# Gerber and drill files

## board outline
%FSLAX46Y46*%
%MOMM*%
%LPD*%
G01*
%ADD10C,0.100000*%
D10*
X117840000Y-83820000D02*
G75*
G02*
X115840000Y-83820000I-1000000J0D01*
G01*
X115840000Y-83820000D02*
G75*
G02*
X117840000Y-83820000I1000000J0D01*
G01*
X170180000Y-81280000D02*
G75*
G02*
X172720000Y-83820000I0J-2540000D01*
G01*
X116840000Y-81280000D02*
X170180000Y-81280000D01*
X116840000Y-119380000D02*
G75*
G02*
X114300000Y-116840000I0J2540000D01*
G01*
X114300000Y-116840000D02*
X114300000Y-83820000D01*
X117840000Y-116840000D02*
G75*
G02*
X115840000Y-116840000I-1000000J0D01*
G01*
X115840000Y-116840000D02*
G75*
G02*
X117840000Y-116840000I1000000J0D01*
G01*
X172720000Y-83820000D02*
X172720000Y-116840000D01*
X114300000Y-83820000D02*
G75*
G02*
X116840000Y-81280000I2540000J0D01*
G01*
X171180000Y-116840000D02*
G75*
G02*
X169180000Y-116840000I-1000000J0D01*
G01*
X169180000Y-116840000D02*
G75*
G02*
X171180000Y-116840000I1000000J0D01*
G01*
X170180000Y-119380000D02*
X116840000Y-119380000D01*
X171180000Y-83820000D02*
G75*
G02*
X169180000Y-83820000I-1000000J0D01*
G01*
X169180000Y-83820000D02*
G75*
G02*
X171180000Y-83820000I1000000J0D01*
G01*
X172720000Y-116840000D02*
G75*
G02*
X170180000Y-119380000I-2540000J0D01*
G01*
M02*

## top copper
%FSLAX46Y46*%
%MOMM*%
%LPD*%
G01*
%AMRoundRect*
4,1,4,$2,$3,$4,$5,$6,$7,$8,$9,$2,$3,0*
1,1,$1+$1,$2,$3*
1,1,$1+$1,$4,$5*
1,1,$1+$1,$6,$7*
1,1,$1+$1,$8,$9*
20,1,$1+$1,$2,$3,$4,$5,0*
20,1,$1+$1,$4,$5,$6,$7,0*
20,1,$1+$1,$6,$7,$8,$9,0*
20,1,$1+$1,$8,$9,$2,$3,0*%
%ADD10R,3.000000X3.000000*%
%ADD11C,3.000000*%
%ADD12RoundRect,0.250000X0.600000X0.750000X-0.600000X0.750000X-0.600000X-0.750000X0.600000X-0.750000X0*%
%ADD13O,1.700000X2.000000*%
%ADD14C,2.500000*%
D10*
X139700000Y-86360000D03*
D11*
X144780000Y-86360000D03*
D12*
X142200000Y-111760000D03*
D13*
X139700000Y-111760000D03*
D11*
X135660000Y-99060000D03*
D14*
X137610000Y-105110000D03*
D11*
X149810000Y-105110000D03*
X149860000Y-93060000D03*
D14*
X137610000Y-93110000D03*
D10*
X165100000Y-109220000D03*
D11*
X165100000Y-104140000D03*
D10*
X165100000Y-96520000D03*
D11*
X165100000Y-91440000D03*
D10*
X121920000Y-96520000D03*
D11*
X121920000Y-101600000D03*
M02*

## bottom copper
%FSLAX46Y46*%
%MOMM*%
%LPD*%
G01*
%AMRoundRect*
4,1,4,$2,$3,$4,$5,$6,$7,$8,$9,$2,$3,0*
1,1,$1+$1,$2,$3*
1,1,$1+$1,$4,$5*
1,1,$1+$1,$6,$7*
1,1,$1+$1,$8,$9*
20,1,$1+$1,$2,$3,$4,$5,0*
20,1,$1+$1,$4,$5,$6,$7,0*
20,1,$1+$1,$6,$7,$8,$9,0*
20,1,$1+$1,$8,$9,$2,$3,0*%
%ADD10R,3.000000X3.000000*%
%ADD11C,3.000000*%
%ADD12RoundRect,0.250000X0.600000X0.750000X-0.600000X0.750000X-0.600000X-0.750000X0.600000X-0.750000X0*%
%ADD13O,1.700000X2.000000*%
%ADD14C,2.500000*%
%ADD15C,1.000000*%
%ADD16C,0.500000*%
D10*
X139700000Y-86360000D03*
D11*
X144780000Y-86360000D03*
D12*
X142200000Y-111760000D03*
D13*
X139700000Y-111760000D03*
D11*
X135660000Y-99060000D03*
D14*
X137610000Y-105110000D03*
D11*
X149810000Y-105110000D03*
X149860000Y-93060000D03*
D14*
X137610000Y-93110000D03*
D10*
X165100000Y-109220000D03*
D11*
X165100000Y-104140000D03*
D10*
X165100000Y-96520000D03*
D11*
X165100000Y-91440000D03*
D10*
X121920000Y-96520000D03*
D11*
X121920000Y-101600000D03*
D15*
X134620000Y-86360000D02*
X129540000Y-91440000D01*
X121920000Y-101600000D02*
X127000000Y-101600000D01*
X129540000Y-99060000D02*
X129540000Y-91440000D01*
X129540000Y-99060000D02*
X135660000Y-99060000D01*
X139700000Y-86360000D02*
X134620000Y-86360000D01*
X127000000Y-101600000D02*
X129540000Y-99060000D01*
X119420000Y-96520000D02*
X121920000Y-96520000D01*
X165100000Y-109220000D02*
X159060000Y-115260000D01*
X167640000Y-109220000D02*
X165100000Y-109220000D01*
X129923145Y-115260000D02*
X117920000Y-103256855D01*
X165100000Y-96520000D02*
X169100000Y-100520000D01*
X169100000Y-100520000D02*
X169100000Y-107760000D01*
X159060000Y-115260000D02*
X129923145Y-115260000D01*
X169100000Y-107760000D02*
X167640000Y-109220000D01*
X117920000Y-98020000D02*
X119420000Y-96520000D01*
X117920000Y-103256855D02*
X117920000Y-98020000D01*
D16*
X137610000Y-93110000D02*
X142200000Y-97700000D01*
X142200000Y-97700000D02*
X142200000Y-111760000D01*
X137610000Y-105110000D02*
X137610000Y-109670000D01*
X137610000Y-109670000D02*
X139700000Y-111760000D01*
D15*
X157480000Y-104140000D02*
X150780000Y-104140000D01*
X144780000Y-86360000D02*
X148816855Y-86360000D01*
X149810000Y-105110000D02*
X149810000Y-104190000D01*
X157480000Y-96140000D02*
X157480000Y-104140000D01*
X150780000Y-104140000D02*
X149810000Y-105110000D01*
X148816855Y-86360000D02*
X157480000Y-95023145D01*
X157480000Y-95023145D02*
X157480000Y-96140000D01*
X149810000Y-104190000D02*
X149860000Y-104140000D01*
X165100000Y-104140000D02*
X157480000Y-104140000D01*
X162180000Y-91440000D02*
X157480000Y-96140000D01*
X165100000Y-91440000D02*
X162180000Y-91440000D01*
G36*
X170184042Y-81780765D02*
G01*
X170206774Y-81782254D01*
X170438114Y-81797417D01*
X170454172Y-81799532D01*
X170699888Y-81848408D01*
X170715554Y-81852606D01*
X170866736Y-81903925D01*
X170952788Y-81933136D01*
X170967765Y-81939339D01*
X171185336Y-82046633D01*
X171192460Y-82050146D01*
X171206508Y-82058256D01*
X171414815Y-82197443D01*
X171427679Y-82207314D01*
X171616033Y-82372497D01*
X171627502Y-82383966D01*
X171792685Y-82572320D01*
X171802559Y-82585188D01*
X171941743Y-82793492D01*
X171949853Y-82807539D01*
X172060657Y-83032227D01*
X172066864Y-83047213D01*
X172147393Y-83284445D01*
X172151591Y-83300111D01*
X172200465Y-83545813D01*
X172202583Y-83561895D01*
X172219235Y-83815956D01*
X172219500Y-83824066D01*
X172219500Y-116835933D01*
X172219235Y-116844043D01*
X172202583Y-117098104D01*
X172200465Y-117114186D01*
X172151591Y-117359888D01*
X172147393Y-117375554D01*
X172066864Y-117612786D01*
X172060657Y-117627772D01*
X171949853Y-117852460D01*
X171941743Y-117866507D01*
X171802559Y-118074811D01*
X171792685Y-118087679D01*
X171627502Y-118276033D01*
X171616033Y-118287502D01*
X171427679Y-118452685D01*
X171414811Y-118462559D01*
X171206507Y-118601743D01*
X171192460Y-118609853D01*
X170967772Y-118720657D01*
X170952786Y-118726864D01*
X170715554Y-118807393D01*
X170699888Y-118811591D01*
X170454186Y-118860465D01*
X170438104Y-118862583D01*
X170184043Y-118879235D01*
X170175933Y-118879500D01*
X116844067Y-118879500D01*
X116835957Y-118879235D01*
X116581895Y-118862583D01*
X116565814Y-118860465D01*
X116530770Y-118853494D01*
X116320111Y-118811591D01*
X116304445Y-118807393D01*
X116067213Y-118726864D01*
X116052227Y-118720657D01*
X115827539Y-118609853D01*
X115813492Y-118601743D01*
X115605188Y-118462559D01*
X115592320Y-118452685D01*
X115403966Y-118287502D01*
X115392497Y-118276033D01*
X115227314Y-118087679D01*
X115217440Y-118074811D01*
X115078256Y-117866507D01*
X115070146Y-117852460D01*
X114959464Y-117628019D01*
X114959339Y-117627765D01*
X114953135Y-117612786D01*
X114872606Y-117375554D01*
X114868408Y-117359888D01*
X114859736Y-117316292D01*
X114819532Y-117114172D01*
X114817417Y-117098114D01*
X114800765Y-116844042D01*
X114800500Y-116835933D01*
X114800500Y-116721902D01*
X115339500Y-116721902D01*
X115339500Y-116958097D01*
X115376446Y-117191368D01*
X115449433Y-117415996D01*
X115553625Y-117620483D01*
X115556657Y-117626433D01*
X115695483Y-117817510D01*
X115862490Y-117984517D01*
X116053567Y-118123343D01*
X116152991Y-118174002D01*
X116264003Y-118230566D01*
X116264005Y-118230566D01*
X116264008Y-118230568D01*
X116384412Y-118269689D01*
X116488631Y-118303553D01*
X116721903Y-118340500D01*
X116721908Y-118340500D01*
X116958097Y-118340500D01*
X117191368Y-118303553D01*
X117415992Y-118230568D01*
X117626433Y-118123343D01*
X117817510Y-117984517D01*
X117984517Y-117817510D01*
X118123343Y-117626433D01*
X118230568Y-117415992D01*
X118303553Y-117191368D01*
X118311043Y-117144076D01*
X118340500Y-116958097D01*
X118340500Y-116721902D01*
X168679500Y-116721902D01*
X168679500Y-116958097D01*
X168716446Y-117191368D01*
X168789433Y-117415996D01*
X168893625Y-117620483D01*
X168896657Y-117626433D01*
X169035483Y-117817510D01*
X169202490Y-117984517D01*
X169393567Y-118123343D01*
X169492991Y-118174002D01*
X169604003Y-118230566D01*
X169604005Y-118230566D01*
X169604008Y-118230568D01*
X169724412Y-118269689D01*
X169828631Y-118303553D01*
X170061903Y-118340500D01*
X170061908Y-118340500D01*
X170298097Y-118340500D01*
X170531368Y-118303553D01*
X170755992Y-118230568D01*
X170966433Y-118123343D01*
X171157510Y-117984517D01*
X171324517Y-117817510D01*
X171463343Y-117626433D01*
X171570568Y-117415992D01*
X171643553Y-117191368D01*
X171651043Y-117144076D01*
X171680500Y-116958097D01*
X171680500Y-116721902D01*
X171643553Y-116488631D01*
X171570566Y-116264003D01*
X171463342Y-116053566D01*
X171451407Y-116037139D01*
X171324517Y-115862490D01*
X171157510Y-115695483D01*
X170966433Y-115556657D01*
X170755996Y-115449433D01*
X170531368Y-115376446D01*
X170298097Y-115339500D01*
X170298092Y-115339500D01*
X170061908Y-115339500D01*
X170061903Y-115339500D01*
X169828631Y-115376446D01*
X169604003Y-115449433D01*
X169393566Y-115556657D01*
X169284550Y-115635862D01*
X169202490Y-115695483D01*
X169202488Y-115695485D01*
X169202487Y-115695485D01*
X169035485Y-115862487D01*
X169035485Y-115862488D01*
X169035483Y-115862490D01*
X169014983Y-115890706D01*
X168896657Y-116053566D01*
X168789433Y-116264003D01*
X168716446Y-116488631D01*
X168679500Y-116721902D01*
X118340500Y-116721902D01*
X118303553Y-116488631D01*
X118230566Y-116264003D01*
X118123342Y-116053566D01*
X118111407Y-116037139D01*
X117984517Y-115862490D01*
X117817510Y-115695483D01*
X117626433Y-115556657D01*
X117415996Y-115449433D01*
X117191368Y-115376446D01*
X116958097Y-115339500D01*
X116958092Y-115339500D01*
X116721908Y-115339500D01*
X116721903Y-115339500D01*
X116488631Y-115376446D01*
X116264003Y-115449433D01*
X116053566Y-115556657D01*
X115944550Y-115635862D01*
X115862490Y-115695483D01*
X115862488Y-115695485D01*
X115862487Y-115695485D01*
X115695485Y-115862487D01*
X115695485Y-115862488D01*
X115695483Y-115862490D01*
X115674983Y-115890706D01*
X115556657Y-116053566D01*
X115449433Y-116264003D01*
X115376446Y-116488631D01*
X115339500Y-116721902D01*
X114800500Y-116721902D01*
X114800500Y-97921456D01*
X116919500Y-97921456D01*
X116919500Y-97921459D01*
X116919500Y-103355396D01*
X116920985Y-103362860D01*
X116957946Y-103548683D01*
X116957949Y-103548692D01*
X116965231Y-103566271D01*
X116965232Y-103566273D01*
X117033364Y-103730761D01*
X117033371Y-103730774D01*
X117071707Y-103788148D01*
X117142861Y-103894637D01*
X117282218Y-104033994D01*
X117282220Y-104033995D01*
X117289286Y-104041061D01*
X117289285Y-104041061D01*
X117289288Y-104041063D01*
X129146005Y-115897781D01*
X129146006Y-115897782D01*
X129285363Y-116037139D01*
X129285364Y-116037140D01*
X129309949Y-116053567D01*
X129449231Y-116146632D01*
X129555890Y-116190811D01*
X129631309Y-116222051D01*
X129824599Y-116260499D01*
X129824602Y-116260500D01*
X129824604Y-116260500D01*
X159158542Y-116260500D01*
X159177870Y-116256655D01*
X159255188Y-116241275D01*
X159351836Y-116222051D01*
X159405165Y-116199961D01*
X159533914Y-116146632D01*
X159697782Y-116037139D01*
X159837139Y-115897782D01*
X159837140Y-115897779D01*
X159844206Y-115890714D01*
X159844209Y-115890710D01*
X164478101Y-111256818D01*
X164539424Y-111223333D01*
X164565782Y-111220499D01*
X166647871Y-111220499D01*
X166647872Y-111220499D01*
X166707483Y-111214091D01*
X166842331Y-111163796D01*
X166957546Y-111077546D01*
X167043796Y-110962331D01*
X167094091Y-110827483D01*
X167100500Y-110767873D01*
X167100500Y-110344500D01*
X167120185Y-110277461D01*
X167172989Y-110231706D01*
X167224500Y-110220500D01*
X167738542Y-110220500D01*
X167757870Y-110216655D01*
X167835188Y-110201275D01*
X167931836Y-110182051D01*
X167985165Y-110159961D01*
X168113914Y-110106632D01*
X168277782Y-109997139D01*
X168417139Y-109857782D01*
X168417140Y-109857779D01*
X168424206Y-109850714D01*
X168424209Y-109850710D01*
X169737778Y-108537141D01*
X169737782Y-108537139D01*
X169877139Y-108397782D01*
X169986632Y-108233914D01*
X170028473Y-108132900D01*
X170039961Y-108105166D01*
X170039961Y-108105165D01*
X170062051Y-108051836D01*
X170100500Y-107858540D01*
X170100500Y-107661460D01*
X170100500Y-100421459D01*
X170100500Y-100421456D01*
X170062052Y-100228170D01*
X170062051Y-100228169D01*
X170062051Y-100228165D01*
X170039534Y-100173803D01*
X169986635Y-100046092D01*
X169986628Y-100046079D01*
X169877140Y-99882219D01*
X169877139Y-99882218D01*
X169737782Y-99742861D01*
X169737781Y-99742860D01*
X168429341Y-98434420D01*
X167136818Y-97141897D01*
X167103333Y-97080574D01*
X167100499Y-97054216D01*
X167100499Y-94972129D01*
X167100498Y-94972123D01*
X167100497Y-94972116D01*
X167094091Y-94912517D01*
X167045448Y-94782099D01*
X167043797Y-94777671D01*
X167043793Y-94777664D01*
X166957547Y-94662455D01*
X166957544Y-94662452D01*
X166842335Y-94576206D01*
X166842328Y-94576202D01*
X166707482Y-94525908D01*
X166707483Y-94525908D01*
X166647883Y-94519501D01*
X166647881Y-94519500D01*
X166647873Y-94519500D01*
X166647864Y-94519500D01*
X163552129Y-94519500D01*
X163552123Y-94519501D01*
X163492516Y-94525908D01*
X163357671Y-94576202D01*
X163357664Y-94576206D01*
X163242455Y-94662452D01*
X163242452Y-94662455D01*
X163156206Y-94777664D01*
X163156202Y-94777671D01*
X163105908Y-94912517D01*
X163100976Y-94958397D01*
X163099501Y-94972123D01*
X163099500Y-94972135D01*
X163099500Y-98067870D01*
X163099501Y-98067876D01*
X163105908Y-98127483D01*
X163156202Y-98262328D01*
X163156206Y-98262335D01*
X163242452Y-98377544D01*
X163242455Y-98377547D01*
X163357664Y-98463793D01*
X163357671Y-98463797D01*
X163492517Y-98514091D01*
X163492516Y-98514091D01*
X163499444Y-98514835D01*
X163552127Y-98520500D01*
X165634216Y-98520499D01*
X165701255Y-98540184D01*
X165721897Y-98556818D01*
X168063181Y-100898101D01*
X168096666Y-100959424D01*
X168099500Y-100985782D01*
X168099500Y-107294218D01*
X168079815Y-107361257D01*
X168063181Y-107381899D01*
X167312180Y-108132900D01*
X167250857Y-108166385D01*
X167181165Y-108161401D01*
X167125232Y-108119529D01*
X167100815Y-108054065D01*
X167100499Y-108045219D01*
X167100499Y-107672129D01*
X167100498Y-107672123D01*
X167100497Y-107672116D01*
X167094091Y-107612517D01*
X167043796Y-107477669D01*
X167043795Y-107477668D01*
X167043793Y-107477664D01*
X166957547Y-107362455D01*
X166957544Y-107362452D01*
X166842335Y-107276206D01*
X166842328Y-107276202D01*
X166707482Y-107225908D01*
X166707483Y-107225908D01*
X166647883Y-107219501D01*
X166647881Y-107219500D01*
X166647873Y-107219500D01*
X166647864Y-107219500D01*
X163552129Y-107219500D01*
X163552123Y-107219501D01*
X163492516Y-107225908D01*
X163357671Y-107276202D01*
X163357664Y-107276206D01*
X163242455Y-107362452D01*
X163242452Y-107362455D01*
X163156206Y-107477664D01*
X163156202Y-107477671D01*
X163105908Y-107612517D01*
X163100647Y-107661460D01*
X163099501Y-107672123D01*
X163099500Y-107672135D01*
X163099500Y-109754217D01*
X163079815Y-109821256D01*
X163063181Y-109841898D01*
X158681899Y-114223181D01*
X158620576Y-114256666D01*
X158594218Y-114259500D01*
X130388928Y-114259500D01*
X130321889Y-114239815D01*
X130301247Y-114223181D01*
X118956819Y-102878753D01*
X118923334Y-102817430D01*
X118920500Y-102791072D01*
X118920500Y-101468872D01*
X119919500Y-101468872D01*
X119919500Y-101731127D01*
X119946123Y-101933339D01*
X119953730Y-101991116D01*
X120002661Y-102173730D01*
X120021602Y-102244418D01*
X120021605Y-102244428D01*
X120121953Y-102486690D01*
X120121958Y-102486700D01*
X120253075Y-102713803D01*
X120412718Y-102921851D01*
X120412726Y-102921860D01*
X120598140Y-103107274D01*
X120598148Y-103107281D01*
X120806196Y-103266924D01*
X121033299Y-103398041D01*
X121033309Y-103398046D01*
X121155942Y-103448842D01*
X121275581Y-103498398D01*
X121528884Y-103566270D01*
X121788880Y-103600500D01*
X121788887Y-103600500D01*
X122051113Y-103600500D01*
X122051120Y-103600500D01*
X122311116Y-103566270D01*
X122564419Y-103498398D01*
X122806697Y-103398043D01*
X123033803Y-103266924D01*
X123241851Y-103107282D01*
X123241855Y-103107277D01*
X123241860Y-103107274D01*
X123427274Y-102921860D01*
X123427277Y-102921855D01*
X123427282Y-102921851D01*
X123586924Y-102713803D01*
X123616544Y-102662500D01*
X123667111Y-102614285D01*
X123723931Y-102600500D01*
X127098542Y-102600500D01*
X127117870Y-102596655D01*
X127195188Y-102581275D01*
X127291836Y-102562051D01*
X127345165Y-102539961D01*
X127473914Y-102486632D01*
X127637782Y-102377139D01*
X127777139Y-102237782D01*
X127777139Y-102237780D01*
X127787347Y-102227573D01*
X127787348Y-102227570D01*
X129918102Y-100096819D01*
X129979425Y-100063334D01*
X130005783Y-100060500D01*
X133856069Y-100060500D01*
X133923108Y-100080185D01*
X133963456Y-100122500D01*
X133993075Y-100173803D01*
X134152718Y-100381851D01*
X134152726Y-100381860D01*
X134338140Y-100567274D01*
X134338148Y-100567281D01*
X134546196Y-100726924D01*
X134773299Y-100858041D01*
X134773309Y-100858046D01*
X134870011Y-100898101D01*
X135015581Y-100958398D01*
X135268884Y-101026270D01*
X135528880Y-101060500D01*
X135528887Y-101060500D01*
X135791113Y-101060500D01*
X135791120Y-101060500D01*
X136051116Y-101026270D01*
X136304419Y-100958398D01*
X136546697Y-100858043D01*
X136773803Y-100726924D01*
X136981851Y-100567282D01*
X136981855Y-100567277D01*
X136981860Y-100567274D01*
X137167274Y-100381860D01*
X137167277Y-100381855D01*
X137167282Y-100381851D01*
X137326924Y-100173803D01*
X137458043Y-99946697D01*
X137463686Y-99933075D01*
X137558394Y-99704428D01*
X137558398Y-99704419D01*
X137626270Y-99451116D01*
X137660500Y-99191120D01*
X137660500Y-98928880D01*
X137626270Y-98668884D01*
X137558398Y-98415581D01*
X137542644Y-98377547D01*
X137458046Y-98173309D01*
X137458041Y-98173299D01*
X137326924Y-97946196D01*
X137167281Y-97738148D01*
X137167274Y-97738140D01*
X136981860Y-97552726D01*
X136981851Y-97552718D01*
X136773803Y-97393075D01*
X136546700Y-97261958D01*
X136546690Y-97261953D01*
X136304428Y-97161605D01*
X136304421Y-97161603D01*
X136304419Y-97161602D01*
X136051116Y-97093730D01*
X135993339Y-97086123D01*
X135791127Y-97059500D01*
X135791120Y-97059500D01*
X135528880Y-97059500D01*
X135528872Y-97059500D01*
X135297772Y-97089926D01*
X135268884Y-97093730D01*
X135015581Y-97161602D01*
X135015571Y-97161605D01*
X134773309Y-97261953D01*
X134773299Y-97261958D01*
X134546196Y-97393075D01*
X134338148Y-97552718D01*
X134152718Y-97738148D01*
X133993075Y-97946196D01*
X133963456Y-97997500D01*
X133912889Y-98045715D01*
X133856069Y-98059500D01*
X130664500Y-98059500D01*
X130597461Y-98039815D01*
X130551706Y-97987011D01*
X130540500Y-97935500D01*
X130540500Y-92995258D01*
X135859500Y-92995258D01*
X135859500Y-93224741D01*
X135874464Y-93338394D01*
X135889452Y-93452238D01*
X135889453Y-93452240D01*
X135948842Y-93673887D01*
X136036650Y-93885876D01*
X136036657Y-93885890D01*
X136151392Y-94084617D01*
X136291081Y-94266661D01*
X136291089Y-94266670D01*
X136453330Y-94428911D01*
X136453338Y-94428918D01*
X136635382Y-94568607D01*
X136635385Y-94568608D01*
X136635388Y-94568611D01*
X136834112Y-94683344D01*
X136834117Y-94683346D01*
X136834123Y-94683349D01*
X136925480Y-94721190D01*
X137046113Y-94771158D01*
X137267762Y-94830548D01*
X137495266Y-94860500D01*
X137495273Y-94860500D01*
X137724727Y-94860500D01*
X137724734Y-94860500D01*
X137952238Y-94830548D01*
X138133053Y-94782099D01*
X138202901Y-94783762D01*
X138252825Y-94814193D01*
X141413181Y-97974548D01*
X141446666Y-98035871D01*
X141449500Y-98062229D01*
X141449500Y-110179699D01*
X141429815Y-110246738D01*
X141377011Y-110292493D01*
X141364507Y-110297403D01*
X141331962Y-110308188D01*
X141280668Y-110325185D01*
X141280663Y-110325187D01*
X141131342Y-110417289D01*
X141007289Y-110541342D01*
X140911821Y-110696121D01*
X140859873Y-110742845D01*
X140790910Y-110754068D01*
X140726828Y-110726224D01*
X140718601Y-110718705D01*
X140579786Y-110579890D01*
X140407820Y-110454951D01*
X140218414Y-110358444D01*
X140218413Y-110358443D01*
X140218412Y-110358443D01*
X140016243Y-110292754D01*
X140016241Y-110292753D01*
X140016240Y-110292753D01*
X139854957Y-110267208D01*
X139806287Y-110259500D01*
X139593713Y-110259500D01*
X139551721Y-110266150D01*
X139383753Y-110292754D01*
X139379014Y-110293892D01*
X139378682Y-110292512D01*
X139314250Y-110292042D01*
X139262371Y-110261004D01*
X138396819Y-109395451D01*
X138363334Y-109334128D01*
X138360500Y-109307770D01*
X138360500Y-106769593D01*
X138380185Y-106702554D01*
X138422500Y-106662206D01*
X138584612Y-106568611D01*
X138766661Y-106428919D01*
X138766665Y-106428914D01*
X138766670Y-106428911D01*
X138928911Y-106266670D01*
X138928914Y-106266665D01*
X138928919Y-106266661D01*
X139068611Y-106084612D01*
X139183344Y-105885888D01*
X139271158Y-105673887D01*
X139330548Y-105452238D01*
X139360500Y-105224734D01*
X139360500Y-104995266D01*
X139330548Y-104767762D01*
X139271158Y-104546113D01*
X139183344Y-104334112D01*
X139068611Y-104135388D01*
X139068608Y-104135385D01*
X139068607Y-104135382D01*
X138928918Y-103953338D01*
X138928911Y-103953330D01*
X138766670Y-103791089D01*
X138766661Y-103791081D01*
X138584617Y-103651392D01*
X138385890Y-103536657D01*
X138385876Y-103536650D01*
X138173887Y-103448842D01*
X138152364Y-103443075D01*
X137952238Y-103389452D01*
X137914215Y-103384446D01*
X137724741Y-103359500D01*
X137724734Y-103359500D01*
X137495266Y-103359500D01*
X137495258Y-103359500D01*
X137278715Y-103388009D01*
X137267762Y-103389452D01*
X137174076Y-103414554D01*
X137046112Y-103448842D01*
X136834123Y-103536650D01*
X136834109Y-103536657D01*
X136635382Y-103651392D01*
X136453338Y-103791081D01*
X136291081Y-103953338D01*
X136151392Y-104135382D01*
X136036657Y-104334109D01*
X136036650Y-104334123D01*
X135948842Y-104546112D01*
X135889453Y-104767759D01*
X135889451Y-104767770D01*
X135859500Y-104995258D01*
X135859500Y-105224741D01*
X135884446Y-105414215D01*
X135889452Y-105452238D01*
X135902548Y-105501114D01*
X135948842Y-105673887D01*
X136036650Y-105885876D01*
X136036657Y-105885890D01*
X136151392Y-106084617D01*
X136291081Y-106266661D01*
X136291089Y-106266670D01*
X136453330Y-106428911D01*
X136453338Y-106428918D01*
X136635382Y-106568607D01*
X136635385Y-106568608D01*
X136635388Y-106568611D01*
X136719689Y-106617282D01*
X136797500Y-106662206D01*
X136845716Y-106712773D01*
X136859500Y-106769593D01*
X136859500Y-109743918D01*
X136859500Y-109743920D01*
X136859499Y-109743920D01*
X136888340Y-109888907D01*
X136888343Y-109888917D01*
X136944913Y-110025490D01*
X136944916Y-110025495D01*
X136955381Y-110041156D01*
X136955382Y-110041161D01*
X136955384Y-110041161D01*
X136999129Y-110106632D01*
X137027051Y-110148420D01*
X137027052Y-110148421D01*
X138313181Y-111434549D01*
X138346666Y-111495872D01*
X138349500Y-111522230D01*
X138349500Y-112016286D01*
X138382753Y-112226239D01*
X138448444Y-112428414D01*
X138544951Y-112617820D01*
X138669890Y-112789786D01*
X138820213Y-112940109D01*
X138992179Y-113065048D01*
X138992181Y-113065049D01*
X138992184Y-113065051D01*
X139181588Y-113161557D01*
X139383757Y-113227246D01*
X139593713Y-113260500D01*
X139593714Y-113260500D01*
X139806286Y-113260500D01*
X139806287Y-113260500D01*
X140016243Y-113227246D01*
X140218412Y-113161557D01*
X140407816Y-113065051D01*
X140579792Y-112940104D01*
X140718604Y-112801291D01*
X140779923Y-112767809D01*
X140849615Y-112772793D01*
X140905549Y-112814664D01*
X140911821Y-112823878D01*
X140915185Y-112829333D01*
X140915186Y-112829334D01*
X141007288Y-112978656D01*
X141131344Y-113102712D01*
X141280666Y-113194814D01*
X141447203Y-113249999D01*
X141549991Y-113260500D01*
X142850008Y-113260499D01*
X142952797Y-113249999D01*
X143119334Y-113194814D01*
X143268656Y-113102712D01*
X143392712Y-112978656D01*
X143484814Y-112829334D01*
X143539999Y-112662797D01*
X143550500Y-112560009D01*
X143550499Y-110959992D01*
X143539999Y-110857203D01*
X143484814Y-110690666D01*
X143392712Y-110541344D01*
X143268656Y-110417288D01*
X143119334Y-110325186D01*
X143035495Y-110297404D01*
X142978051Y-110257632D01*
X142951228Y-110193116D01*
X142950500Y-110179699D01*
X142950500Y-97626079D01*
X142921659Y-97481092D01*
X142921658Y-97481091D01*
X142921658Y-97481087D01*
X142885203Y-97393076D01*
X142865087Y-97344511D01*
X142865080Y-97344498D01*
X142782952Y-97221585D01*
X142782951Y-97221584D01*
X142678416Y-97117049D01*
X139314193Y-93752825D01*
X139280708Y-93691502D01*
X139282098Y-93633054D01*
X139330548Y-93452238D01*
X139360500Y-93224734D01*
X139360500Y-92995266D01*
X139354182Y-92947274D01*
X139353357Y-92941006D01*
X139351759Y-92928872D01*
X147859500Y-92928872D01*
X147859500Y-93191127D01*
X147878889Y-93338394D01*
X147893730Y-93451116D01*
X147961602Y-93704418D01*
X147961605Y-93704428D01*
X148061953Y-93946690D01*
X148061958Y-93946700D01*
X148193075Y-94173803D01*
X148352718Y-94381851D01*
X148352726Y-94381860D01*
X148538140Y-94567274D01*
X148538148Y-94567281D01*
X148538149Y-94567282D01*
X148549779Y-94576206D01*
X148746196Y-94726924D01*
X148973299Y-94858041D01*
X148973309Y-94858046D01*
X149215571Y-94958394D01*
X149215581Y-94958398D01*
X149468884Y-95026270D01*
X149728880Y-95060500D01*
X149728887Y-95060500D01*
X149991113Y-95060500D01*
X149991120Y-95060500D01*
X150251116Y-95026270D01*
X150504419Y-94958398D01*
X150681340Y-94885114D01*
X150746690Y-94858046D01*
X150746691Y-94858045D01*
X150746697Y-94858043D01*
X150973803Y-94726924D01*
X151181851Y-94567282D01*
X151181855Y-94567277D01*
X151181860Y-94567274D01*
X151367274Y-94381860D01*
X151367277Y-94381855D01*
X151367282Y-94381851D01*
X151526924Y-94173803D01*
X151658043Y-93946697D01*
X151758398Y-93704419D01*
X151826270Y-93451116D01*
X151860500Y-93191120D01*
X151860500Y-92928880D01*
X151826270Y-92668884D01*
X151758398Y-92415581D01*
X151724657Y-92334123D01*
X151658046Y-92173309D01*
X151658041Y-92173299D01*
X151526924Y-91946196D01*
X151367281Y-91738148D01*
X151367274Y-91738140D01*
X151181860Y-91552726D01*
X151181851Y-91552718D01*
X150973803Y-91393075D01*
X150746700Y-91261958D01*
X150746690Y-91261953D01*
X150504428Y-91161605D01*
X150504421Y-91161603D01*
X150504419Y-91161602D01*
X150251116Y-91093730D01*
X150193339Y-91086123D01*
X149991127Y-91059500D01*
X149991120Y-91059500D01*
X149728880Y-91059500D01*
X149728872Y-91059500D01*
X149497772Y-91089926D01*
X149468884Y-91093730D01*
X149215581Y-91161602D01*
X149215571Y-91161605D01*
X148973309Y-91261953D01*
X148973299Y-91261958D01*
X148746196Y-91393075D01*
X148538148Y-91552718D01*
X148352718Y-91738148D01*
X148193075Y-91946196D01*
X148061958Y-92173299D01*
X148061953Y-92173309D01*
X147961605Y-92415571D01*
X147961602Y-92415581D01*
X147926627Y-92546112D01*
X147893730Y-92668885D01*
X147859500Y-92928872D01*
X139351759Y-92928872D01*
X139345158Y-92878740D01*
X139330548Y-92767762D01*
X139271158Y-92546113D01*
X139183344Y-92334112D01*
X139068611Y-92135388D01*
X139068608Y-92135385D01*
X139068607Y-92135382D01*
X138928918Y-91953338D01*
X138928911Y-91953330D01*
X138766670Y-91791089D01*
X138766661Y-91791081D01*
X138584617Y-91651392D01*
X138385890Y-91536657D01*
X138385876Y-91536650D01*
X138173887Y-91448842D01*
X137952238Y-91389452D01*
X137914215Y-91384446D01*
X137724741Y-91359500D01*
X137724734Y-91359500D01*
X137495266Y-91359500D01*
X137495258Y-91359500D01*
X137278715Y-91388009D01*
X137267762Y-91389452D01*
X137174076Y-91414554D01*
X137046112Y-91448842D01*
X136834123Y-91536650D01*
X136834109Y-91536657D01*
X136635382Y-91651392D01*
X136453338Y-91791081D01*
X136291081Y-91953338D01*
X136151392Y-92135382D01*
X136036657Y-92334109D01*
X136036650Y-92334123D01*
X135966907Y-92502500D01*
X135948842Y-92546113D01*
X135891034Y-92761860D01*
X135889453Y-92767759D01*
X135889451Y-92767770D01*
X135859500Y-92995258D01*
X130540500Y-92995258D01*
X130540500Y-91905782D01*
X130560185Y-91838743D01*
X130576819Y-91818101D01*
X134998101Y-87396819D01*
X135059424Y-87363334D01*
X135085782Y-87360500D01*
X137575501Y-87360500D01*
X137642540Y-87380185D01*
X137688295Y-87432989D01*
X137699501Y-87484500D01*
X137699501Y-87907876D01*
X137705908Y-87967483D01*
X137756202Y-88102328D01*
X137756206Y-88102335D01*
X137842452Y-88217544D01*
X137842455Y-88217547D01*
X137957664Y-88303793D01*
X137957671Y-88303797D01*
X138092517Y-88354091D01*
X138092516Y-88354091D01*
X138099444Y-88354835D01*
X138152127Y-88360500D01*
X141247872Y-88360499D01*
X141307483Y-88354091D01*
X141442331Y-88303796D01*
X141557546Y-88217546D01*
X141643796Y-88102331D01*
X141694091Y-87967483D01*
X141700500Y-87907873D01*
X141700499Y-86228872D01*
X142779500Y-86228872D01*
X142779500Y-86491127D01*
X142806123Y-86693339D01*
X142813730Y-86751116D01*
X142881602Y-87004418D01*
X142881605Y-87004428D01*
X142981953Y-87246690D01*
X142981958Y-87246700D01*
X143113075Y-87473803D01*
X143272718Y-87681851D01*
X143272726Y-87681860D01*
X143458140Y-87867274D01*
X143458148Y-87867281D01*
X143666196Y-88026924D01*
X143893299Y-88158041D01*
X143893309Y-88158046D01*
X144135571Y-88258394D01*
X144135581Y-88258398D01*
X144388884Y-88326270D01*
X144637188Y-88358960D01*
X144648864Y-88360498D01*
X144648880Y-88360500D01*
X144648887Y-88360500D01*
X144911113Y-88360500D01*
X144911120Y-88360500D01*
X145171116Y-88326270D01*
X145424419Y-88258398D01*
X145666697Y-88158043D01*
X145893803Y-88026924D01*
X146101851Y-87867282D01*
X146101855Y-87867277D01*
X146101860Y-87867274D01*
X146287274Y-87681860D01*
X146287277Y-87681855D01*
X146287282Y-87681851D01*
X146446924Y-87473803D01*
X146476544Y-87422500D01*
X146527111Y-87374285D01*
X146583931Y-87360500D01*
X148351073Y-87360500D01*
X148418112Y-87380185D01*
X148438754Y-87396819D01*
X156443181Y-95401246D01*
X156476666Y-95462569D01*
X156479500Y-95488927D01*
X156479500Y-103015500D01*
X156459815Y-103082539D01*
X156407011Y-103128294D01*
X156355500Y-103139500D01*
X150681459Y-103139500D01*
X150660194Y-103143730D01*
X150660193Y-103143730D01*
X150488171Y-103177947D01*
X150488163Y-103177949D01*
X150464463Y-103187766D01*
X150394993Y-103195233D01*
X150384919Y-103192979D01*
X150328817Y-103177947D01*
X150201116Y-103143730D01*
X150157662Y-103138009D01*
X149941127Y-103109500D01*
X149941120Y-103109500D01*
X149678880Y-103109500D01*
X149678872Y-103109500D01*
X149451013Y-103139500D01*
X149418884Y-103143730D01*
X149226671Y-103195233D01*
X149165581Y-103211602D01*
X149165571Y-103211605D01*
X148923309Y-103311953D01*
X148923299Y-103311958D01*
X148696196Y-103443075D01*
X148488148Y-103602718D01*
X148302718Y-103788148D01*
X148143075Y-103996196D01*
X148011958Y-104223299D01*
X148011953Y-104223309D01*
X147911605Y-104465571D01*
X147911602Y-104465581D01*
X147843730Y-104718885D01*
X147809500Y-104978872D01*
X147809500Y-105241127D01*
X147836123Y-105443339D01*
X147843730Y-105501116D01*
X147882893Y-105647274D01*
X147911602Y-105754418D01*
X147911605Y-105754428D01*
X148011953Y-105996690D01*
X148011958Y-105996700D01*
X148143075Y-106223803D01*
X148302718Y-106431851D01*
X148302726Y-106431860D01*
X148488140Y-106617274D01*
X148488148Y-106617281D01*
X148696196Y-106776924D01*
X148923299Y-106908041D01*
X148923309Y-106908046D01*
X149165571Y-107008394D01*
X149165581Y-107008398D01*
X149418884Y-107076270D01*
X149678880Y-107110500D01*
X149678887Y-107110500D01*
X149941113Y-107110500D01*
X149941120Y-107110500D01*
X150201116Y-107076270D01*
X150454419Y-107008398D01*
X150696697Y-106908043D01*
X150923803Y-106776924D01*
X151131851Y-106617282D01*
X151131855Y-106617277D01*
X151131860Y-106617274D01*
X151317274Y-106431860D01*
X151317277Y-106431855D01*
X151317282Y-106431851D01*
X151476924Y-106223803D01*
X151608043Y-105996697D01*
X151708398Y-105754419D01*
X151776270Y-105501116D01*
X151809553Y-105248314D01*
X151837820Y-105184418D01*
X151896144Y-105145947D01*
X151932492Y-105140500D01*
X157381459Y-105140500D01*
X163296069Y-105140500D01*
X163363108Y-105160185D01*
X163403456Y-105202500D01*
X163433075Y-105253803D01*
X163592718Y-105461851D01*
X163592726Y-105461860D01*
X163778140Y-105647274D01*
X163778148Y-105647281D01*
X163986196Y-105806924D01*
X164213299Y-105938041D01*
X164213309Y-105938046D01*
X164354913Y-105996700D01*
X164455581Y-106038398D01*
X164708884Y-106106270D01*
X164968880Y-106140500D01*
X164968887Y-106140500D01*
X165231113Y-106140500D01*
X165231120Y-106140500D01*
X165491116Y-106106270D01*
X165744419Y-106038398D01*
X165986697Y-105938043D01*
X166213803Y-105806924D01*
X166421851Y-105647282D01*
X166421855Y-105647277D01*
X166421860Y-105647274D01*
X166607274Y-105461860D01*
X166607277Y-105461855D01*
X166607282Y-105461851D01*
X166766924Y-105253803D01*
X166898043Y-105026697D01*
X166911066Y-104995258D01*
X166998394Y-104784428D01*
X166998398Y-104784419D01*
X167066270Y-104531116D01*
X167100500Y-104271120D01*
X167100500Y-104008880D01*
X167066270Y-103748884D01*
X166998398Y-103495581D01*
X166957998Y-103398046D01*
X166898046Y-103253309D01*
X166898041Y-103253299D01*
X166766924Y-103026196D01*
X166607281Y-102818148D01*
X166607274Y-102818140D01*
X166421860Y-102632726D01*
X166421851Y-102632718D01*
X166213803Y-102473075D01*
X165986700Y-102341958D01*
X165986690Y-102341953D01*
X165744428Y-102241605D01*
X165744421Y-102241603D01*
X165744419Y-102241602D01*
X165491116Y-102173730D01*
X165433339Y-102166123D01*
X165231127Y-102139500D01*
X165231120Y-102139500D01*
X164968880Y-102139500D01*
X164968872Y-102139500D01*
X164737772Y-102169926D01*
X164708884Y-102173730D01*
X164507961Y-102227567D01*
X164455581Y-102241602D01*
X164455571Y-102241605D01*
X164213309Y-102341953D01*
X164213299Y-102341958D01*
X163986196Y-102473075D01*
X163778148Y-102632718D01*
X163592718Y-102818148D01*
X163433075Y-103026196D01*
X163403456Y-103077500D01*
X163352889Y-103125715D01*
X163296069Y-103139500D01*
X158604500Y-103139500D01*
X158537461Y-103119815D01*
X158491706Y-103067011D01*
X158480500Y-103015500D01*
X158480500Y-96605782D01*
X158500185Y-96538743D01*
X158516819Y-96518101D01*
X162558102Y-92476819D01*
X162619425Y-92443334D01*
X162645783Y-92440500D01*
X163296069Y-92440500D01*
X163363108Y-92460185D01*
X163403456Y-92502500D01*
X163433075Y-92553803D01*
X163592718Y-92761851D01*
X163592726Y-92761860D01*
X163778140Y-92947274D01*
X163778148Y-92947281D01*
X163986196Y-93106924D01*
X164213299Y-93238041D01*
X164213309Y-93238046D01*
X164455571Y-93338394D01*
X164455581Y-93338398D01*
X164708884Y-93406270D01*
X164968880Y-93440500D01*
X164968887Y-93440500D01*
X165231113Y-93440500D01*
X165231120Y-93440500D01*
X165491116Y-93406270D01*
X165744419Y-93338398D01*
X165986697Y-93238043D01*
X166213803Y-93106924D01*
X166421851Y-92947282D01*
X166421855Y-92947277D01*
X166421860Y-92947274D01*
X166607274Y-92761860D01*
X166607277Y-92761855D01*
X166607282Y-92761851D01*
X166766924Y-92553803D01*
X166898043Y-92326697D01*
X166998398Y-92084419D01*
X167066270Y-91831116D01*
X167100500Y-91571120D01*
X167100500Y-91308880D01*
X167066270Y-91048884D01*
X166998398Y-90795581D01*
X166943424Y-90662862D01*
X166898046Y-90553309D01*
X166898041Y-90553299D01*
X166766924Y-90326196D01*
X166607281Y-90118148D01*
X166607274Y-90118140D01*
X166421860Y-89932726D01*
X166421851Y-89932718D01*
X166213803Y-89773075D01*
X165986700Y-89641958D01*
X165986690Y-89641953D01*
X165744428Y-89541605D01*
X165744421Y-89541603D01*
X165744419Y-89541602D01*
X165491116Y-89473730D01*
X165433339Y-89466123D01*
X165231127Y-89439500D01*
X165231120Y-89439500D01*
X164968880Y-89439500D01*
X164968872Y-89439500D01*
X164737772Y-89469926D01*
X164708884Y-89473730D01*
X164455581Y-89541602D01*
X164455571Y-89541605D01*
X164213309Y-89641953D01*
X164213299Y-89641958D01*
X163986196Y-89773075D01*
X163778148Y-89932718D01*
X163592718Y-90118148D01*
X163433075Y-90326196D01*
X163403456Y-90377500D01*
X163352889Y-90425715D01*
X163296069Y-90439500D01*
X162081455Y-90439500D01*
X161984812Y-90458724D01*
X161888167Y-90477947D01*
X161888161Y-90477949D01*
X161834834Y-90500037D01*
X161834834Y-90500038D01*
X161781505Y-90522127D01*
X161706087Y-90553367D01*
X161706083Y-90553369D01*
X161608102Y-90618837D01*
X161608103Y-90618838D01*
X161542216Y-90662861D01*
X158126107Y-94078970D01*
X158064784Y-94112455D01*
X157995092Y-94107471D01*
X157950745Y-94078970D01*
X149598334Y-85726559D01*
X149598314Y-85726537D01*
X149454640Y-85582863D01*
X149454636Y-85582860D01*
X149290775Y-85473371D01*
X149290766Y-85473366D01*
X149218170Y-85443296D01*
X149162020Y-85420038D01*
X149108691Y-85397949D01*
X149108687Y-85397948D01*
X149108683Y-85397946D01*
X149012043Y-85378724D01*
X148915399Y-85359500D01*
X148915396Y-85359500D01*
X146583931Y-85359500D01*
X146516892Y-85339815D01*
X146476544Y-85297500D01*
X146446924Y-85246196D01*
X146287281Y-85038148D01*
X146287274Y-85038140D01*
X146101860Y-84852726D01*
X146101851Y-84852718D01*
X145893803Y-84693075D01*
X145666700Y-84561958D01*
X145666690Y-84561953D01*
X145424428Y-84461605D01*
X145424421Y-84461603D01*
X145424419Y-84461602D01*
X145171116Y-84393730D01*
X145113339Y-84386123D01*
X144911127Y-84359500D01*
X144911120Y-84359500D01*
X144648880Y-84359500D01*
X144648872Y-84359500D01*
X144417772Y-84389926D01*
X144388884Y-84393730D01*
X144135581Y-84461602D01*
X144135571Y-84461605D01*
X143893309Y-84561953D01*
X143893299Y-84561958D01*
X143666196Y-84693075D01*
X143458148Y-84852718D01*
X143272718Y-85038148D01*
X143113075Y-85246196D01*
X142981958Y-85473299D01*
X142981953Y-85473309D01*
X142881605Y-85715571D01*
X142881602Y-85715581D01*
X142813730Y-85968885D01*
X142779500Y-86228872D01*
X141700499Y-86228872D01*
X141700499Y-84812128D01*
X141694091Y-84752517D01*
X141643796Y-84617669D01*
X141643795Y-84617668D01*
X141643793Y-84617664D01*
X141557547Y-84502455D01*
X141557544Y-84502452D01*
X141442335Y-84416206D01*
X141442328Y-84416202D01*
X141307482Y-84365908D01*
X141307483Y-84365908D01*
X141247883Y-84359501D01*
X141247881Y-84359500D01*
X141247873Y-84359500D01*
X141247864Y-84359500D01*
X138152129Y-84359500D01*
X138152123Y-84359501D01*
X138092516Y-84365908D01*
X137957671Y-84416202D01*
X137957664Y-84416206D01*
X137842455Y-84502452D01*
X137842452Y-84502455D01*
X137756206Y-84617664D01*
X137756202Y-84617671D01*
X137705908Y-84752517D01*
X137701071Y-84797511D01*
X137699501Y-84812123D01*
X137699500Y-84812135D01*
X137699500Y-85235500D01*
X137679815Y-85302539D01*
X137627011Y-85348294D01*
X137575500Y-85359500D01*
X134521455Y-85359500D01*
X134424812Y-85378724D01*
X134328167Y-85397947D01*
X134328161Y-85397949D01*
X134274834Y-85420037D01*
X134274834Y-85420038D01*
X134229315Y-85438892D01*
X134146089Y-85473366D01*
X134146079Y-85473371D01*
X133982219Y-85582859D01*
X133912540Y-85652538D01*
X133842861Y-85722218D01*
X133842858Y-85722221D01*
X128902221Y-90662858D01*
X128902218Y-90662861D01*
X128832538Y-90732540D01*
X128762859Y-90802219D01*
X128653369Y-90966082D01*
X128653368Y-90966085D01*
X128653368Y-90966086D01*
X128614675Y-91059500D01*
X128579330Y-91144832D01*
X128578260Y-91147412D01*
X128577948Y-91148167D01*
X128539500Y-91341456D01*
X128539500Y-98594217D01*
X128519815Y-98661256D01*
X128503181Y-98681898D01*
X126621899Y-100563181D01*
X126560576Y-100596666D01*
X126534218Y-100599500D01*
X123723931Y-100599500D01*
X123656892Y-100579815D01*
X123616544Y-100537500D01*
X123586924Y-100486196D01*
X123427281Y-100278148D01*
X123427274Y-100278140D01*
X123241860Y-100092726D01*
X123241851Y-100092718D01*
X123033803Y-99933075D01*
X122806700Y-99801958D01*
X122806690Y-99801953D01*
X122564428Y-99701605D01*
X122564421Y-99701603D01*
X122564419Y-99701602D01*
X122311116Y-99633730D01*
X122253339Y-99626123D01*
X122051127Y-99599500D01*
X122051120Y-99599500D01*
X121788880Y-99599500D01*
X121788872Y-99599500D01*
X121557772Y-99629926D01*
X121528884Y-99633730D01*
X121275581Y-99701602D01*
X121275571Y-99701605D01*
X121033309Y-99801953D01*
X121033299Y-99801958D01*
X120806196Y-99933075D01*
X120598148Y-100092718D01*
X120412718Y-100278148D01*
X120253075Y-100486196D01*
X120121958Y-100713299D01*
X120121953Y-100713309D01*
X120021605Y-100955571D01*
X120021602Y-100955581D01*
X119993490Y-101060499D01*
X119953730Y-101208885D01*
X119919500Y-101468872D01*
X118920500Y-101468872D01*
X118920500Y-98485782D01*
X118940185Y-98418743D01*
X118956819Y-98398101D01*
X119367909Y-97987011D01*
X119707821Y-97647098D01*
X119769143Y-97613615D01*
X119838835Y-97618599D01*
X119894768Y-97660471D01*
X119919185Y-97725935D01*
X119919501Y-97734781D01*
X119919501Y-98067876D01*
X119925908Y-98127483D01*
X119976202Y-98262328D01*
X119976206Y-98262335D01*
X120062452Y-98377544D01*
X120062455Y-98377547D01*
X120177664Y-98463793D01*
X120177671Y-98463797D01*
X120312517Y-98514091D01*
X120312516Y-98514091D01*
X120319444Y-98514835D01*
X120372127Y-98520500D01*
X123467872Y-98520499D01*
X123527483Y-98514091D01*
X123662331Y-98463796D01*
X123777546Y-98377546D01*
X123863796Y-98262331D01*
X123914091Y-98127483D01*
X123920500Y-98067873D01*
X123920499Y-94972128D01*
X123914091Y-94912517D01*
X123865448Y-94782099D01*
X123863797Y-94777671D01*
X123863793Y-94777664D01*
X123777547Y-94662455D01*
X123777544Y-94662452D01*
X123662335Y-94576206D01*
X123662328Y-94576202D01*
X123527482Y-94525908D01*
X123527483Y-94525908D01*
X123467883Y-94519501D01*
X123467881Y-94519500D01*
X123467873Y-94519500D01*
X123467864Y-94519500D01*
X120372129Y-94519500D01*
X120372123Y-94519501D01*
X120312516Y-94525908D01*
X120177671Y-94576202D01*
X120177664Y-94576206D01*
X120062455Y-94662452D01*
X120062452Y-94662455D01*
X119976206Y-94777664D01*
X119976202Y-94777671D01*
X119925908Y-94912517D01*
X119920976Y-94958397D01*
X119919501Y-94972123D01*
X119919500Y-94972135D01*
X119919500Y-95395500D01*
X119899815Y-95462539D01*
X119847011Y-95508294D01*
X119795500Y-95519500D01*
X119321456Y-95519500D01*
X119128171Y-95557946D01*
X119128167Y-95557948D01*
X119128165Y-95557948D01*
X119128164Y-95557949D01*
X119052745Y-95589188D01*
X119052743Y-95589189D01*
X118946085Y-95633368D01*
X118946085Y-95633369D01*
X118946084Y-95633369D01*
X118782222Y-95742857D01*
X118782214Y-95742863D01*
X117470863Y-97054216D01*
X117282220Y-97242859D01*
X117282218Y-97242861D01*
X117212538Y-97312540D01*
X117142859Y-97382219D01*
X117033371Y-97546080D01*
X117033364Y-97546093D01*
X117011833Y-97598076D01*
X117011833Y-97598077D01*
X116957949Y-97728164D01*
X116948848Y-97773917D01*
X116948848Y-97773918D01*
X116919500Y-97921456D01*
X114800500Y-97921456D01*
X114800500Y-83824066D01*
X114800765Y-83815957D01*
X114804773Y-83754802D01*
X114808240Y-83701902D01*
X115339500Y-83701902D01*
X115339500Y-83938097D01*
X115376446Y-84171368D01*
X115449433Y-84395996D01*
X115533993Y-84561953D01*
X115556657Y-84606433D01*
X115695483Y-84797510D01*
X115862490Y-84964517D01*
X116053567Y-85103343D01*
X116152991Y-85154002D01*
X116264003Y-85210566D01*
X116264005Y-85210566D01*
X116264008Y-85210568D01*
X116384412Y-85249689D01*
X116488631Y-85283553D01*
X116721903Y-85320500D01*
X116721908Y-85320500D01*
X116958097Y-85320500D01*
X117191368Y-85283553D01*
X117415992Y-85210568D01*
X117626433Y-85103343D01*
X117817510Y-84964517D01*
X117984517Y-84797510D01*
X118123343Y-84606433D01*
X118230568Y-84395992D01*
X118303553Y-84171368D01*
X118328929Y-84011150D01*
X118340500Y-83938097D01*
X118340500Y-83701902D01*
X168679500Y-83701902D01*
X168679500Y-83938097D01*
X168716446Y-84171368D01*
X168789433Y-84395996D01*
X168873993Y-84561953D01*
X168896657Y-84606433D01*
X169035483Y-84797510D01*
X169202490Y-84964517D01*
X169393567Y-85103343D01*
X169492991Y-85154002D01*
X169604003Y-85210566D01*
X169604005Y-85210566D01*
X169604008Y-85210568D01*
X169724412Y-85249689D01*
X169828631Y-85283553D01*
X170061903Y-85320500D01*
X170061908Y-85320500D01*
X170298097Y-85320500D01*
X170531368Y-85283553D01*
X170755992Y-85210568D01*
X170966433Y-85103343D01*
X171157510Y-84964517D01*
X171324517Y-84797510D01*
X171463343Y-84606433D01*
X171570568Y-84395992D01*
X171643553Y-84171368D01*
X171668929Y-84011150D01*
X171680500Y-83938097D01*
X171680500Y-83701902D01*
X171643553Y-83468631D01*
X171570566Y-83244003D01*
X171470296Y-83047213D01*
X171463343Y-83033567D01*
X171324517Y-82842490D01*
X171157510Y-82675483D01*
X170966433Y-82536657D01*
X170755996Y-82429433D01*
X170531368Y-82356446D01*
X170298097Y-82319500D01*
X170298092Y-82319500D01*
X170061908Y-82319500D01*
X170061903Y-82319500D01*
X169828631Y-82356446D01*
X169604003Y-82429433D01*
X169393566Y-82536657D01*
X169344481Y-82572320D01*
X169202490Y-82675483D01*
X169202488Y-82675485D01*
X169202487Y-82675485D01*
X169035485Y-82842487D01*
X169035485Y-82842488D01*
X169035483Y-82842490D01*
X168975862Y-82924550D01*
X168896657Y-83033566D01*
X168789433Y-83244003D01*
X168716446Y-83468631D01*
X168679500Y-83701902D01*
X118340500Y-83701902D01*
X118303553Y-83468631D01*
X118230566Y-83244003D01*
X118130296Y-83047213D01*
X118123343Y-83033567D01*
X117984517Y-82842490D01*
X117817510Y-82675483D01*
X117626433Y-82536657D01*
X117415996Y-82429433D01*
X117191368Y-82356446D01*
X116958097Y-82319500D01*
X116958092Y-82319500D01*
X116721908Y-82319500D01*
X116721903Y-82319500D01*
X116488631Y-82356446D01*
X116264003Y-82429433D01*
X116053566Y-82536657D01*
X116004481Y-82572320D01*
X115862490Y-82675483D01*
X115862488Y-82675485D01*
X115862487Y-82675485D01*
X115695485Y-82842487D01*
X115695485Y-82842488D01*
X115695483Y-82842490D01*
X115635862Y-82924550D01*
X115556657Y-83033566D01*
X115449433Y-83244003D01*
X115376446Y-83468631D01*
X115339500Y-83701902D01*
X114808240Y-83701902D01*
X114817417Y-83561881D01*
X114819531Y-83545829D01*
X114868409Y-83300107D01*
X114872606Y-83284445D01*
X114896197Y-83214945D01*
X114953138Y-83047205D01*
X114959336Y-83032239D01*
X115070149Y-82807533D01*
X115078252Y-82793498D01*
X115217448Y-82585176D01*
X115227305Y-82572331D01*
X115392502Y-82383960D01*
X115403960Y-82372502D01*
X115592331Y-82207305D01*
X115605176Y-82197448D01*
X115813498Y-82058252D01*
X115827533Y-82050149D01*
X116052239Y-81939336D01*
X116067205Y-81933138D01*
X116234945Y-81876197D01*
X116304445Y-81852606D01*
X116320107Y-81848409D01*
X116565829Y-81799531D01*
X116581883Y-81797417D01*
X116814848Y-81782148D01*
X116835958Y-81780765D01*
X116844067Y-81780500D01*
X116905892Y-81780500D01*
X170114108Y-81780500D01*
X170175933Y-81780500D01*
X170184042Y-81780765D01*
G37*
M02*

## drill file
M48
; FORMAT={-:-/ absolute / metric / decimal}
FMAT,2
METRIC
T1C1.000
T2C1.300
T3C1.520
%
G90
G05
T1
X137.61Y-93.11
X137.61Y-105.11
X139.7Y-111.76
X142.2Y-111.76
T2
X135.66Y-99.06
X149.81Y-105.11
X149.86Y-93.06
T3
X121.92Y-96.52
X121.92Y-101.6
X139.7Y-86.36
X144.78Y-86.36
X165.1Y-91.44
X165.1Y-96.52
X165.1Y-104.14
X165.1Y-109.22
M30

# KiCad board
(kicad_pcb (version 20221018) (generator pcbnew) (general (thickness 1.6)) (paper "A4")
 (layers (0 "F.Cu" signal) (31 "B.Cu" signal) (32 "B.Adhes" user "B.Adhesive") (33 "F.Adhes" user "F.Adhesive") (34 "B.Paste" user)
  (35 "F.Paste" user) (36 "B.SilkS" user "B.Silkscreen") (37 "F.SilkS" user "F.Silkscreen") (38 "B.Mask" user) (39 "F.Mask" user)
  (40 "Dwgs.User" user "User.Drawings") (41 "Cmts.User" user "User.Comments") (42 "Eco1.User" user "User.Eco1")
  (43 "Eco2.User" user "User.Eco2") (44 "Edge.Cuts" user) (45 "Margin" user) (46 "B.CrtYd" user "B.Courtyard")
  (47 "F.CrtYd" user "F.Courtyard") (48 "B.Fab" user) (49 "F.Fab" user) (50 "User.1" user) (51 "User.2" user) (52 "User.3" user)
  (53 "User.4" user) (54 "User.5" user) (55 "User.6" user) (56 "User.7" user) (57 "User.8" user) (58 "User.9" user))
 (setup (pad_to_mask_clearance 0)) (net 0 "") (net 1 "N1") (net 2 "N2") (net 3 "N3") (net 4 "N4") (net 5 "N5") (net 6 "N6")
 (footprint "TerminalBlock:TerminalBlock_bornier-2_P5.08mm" (layer "F.Cu") (at 139.7 86.36)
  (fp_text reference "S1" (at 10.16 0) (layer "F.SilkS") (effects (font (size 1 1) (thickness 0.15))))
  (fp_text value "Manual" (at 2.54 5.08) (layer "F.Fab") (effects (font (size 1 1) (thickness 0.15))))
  (pad "1" thru_hole rect (at 0 0) (size 3 3) (drill 1.52) (layers "*.Cu" "*.Mask") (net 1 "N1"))
  (pad "2" thru_hole circle (at 5.08 0) (size 3 3) (drill 1.52) (layers "*.Cu" "*.Mask") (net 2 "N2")))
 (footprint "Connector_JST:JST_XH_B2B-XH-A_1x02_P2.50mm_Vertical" (layer "F.Cu") (at 142.2 111.76 180)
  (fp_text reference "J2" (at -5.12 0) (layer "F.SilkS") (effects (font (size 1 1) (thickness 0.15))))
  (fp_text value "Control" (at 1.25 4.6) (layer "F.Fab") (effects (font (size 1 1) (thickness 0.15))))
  (pad "1" thru_hole roundrect (at 0 0 180) (size 1.7 2) (drill 1) (layers "*.Cu" "*.Mask") (roundrect_rratio 0.147059) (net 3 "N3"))
  (pad "2" thru_hole oval (at 2.5 0 180) (size 1.7 2) (drill 1) (layers "*.Cu" "*.Mask") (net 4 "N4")))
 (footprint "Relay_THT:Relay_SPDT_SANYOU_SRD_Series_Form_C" (layer "F.Cu") (at 135.66 99.06)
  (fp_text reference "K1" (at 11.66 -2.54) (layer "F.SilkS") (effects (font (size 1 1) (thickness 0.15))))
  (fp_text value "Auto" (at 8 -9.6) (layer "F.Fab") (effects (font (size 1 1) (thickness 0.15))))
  (pad "1" thru_hole circle (at 0 0 90) (size 3 3) (drill 1.3) (layers "*.Cu" "*.Mask") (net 1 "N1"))
  (pad "2" thru_hole circle (at 1.95 6.05 90) (size 2.5 2.5) (drill 1) (layers "*.Cu" "*.Mask") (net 4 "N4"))
  (pad "3" thru_hole circle (at 14.15 6.05 90) (size 3 3) (drill 1.3) (layers "*.Cu" "*.Mask") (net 2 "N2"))
  (pad "4" thru_hole circle (at 14.2 -6 90) (size 3 3) (drill 1.3) (layers "*.Cu" "*.Mask") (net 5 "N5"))
  (pad "5" thru_hole circle (at 1.95 -5.95 90) (size 2.5 2.5) (drill 1) (layers "*.Cu" "*.Mask") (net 3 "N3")))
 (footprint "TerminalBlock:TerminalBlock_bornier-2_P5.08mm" (layer "F.Cu") (at 165.1 109.22 90)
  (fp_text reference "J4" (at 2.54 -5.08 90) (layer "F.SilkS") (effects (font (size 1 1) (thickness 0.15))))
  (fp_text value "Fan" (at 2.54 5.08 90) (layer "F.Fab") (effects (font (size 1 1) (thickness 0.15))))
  (pad "1" thru_hole rect (at 0 0 90) (size 3 3) (drill 1.52) (layers "*.Cu" "*.Mask") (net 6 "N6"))
  (pad "2" thru_hole circle (at 5.08 0 90) (size 3 3) (drill 1.52) (layers "*.Cu" "*.Mask") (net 2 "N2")))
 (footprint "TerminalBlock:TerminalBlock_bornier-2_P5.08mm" (layer "F.Cu") (at 165.1 96.52 90)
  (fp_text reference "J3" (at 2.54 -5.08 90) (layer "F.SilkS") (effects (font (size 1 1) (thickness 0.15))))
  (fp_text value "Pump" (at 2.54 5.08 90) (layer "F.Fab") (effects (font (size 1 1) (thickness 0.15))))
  (pad "1" thru_hole rect (at 0 0 90) (size 3 3) (drill 1.52) (layers "*.Cu" "*.Mask") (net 6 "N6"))
  (pad "2" thru_hole circle (at 5.08 0 90) (size 3 3) (drill 1.52) (layers "*.Cu" "*.Mask") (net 2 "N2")))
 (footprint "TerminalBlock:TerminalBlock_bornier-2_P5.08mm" (layer "F.Cu") (at 121.92 96.52 -90)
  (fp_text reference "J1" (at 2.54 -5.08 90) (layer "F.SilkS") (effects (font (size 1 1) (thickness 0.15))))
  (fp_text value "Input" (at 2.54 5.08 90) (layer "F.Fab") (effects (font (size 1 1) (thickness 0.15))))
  (pad "1" thru_hole rect (at 0 0 270) (size 3 3) (drill 1.52) (layers "*.Cu" "*.Mask") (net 6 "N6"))
  (pad "2" thru_hole circle (at 5.08 0 270) (size 3 3) (drill 1.52) (layers "*.Cu" "*.Mask") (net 1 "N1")))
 (gr_circle (center 116.84 83.82) (end 117.84 83.82) (stroke (width 0.1) (type default)) (fill none) (layer "Edge.Cuts"))
 (gr_arc (start 170.18 81.28) (mid 171.976051 82.023949) (end 172.72 83.82) (stroke (width 0.1) (type default)) (layer "Edge.Cuts"))
 (gr_line (start 116.84 81.28) (end 170.18 81.28) (stroke (width 0.1) (type default)) (layer "Edge.Cuts"))
 (gr_arc (start 116.84 119.38) (mid 115.043949 118.636051) (end 114.3 116.84) (stroke (width 0.1) (type default)) (layer "Edge.Cuts"))
 (gr_line (start 114.3 116.84) (end 114.3 83.82) (stroke (width 0.1) (type default)) (layer "Edge.Cuts"))
 (gr_circle (center 116.84 116.84) (end 117.84 116.84) (stroke (width 0.1) (type default)) (fill none) (layer "Edge.Cuts"))
 (gr_line (start 172.72 83.82) (end 172.72 116.84) (stroke (width 0.1) (type default)) (layer "Edge.Cuts"))
 (gr_arc (start 114.3 83.82) (mid 115.043949 82.023949) (end 116.84 81.28) (stroke (width 0.1) (type default)) (layer "Edge.Cuts"))
 (gr_circle (center 170.18 116.84) (end 171.18 116.84) (stroke (width 0.1) (type default)) (fill none) (layer "Edge.Cuts"))
 (gr_line (start 170.18 119.38) (end 116.84 119.38) (stroke (width 0.1) (type default)) (layer "Edge.Cuts"))
 (gr_circle (center 170.18 83.82) (end 171.18 83.82) (stroke (width 0.1) (type default)) (fill none) (layer "Edge.Cuts"))
 (gr_arc (start 172.72 116.84) (mid 171.976051 118.636051) (end 170.18 119.38) (stroke (width 0.1) (type default)) (layer "Edge.Cuts"))
 (segment (start 134.62 86.36) (end 129.54 91.44) (width 1) (layer "B.Cu") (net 1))
 (segment (start 121.92 101.6) (end 127 101.6) (width 1) (layer "B.Cu") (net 1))
 (segment (start 129.54 99.06) (end 129.54 91.44) (width 1) (layer "B.Cu") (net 1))
 (segment (start 129.54 99.06) (end 135.66 99.06) (width 1) (layer "B.Cu") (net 1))
 (segment (start 139.7 86.36) (end 134.62 86.36) (width 1) (layer "B.Cu") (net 1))
 (segment (start 127 101.6) (end 129.54 99.06) (width 1) (layer "B.Cu") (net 1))
 (segment (start 119.42 96.52) (end 121.92 96.52) (width 1) (layer "B.Cu") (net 6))
 (segment (start 165.1 109.22) (end 159.06 115.26) (width 1) (layer "B.Cu") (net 6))
 (segment (start 167.64 109.22) (end 165.1 109.22) (width 1) (layer "B.Cu") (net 6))
 (segment (start 129.923145 115.26) (end 117.92 103.256855) (width 1) (layer "B.Cu") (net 6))
 (segment (start 165.1 96.52) (end 169.1 100.52) (width 1) (layer "B.Cu") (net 6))
 (segment (start 169.1 100.52) (end 169.1 107.76) (width 1) (layer "B.Cu") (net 6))
 (segment (start 159.06 115.26) (end 129.923145 115.26) (width 1) (layer "B.Cu") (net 6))
 (segment (start 169.1 107.76) (end 167.64 109.22) (width 1) (layer "B.Cu") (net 6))
 (segment (start 117.92 98.02) (end 119.42 96.52) (width 1) (layer "B.Cu") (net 6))
 (segment (start 117.92 103.256855) (end 117.92 98.02) (width 1) (layer "B.Cu") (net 6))
 (segment (start 137.61 93.11) (end 142.2 97.7) (width 0.5) (layer "B.Cu") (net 3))
 (segment (start 142.2 97.7) (end 142.2 111.76) (width 0.5) (layer "B.Cu") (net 3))
 (segment (start 137.61 105.11) (end 137.61 109.67) (width 0.5) (layer "B.Cu") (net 4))
 (segment (start 137.61 109.67) (end 139.7 111.76) (width 0.5) (layer "B.Cu") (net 4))
 (segment (start 157.48 104.14) (end 150.78 104.14) (width 1) (layer "B.Cu") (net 2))
 (segment (start 144.78 86.36) (end 148.816855 86.36) (width 1) (layer "B.Cu") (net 2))
 (segment (start 149.81 105.11) (end 149.81 104.19) (width 1) (layer "B.Cu") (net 2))
 (segment (start 157.48 96.14) (end 157.48 104.14) (width 1) (layer "B.Cu") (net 2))
 (segment (start 150.78 104.14) (end 149.81 105.11) (width 1) (layer "B.Cu") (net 2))
 (segment (start 148.816855 86.36) (end 157.48 95.023145) (width 1) (layer "B.Cu") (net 2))
 (segment (start 157.48 95.023145) (end 157.48 96.14) (width 1) (layer "B.Cu") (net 2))
 (segment (start 149.81 104.19) (end 149.86 104.14) (width 1) (layer "B.Cu") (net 2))
 (segment (start 165.1 104.14) (end 157.48 104.14) (width 1) (layer "B.Cu") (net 2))
 (segment (start 162.18 91.44) (end 157.48 96.14) (width 1) (layer "B.Cu") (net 2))
 (segment (start 165.1 91.44) (end 162.18 91.44) (width 1) (layer "B.Cu") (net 2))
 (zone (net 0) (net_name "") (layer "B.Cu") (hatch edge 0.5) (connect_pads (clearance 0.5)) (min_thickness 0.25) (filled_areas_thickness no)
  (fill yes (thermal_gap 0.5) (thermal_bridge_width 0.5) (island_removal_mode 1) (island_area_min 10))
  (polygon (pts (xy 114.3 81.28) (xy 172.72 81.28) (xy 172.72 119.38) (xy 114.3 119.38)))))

